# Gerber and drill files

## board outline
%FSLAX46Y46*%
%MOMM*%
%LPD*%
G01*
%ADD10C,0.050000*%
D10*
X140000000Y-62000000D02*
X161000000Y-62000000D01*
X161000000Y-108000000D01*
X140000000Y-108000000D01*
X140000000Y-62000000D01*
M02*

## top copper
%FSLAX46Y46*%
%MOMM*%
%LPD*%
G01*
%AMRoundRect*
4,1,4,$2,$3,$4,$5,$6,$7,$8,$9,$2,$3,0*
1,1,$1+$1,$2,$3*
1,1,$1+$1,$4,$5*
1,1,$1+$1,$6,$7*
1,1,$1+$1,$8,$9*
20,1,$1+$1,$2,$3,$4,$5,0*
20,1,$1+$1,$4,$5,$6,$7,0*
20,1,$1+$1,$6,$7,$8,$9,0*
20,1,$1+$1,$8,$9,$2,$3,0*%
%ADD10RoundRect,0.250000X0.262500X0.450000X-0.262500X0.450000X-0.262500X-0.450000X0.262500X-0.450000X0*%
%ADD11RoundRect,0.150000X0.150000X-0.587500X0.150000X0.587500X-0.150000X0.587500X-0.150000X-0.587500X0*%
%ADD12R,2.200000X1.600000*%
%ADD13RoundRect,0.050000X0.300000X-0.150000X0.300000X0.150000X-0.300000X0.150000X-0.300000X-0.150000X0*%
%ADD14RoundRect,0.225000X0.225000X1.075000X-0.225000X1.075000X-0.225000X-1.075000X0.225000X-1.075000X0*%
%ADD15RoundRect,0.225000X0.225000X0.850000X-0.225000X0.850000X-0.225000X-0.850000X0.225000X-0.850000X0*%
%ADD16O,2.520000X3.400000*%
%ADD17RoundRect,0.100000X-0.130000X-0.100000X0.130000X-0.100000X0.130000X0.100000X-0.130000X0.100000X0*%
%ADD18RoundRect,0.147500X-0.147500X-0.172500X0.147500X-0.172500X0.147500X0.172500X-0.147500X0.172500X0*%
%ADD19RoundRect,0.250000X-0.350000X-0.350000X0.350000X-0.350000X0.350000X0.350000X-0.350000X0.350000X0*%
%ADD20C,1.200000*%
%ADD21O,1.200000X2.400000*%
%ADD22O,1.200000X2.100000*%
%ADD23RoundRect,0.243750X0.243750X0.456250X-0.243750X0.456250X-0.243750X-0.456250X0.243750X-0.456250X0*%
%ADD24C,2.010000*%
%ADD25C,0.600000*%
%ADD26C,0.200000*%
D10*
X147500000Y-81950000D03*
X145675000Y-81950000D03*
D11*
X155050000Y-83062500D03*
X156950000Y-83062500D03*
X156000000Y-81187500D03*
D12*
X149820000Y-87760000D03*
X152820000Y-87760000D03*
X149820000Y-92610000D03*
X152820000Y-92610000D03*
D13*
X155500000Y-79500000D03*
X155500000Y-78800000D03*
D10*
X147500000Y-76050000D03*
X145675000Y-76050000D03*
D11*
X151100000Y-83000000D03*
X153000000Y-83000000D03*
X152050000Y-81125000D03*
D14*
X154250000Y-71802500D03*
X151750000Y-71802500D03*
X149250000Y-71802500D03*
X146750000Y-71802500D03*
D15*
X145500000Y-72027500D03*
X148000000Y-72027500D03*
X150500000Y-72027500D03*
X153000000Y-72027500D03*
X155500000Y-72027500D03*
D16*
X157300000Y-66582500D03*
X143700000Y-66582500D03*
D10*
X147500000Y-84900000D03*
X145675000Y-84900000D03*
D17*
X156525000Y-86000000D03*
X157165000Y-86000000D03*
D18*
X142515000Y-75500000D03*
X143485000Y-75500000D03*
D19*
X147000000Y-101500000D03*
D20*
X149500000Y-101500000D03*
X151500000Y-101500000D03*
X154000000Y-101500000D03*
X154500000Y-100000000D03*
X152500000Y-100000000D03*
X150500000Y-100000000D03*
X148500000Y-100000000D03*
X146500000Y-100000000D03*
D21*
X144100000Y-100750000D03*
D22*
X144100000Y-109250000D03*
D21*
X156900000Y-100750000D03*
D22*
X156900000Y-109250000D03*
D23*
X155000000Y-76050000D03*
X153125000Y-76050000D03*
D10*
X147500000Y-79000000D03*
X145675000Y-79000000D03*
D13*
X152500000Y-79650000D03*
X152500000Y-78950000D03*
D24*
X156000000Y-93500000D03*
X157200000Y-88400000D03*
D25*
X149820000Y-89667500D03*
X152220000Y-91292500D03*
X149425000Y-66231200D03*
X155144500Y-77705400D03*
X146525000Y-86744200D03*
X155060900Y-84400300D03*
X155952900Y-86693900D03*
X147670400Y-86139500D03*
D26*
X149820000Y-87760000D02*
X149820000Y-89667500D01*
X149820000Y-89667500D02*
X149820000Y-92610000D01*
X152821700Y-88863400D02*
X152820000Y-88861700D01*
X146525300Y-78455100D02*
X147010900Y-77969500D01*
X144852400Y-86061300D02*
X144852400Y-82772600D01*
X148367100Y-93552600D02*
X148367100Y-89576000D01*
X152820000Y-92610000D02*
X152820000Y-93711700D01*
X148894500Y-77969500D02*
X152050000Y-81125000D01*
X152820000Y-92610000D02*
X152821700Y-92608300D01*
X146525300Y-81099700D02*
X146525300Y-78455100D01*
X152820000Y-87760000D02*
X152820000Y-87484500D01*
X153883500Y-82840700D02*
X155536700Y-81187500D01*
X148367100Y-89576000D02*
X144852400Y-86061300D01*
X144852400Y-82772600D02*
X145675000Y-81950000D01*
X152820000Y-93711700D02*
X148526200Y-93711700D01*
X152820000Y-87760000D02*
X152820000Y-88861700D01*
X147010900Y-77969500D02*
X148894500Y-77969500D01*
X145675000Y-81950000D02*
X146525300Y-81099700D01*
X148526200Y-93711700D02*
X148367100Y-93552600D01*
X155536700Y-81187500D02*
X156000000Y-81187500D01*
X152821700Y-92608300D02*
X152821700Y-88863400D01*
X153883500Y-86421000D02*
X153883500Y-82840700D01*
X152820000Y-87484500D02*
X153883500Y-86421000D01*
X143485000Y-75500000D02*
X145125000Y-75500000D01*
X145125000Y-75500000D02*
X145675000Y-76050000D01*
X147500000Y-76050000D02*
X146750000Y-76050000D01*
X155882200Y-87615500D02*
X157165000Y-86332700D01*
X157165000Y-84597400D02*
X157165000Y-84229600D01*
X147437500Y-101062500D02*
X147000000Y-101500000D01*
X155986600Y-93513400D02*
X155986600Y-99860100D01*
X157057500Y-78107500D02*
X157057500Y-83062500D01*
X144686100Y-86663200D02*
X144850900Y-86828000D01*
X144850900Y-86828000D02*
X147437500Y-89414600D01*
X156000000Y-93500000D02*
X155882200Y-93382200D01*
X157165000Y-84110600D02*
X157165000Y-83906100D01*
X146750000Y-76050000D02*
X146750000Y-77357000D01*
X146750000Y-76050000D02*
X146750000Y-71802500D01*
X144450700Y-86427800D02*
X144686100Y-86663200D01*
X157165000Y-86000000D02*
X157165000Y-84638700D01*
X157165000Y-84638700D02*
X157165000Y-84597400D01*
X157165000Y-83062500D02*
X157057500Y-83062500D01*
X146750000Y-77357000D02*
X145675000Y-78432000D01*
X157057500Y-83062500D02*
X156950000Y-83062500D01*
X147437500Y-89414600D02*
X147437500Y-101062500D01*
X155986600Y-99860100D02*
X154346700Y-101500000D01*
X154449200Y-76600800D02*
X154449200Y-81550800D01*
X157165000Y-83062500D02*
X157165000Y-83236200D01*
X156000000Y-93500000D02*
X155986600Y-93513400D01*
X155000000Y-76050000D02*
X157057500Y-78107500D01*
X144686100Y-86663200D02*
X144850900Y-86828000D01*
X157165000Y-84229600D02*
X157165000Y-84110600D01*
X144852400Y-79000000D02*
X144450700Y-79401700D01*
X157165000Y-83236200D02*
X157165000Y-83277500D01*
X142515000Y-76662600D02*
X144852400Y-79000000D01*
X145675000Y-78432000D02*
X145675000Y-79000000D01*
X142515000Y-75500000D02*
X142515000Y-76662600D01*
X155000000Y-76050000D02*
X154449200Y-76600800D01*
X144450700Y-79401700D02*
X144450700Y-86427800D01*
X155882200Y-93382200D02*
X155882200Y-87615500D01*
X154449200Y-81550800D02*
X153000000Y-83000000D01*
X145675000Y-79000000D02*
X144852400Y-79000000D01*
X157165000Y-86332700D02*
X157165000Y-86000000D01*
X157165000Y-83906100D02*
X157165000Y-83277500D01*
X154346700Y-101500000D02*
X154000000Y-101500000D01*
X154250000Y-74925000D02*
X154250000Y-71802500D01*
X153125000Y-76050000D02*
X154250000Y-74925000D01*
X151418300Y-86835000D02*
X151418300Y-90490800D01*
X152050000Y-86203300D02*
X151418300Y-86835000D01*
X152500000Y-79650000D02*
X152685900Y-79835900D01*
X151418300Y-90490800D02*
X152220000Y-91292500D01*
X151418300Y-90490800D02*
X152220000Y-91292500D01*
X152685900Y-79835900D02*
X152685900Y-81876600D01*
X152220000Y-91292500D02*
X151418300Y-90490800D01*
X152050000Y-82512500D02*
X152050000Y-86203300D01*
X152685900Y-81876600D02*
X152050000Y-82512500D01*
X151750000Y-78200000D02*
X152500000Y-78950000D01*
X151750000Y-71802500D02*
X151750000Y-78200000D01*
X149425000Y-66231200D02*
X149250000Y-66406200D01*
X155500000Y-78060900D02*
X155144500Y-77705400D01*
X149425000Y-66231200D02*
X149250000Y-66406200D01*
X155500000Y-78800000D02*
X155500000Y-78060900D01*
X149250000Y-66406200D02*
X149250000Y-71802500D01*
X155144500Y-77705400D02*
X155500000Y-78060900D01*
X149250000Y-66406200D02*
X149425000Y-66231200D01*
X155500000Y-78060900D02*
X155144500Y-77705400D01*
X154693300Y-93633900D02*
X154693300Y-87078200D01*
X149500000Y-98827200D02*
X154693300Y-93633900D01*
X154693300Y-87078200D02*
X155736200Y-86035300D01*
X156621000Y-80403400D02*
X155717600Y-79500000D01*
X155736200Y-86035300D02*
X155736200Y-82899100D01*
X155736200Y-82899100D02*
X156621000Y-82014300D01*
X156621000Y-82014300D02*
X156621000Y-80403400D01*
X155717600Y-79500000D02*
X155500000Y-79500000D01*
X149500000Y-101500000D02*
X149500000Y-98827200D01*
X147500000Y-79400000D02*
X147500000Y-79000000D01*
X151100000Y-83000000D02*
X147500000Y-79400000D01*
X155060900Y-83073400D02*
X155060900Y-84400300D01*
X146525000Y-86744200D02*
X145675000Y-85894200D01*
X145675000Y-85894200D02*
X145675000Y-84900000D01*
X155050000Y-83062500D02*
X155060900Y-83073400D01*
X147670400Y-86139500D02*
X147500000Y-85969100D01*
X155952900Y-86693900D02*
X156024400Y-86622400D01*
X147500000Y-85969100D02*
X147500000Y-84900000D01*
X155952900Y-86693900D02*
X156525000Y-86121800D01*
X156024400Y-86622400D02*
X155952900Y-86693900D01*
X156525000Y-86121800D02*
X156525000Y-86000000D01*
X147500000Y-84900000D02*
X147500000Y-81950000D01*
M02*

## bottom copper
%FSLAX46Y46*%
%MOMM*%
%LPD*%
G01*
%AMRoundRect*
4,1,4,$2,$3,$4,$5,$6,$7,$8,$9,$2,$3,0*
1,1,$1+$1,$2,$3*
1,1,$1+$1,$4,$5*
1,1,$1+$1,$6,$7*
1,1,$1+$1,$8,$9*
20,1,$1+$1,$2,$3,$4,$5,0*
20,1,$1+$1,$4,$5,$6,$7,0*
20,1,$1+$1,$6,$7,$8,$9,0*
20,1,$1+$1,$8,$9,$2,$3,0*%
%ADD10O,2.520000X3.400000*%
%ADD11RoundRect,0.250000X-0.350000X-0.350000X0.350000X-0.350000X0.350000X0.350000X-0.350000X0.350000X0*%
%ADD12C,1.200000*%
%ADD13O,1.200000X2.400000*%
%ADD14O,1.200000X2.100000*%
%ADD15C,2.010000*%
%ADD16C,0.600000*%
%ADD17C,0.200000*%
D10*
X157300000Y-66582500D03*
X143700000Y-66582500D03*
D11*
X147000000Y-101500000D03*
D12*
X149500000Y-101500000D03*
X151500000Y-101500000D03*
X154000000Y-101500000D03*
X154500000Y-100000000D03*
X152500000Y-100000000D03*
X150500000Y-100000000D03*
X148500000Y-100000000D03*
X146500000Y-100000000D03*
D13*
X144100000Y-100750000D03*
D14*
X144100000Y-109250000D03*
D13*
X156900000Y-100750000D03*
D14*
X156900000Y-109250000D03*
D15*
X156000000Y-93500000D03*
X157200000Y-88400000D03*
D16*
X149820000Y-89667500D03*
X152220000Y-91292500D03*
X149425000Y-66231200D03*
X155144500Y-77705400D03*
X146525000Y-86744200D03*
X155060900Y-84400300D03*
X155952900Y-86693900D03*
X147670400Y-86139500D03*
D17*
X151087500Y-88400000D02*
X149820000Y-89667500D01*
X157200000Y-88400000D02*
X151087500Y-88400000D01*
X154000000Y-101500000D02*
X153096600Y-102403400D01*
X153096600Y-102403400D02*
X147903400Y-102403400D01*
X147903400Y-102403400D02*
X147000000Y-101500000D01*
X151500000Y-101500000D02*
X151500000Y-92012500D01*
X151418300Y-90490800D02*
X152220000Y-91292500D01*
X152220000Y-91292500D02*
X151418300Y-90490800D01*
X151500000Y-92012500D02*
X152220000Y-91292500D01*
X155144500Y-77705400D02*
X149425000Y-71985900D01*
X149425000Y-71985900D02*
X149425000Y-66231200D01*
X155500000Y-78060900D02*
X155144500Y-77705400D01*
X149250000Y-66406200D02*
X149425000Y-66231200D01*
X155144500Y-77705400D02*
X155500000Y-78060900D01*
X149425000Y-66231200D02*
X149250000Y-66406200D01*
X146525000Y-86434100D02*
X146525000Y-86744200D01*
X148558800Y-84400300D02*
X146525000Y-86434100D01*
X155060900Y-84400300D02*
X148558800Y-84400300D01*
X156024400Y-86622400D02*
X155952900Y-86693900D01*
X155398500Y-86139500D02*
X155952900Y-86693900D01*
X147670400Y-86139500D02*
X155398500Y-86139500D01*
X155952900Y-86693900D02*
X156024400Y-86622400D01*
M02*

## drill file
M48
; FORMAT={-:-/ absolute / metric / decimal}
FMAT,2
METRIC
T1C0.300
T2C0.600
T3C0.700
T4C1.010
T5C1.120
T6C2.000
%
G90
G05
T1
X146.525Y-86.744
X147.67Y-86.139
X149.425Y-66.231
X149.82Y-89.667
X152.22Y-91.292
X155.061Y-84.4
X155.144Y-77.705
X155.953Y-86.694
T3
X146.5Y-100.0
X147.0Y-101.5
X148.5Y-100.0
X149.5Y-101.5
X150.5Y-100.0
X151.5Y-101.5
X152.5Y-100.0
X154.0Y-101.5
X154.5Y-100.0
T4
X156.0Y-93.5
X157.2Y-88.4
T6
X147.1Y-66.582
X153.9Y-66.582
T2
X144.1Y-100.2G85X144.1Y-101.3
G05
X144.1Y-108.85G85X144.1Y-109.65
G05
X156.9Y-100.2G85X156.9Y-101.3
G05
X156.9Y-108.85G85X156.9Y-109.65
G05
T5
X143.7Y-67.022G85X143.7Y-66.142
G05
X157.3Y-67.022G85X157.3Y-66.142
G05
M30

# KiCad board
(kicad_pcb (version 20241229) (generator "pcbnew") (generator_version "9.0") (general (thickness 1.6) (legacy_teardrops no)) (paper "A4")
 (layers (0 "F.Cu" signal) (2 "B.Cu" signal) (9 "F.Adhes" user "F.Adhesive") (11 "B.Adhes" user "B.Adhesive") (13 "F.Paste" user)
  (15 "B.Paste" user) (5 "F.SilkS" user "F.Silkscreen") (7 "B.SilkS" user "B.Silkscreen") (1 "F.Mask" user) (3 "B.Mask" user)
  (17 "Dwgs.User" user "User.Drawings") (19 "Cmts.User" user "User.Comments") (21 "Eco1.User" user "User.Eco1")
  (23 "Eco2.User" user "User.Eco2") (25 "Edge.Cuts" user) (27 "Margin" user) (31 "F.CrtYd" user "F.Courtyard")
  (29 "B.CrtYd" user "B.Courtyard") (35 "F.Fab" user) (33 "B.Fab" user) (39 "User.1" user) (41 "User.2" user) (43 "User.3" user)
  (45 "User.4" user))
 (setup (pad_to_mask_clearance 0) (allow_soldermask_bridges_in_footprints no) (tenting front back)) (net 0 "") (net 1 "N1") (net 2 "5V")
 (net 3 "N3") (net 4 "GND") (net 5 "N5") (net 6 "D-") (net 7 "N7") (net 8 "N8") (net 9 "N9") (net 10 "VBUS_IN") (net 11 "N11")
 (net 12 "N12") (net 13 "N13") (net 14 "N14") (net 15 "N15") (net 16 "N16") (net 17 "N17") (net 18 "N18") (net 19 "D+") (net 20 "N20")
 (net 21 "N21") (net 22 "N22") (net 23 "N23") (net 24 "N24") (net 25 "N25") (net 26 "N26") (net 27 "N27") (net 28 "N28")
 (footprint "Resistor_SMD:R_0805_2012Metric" (layer "F.Cu") (at 146.5875 81.95 180)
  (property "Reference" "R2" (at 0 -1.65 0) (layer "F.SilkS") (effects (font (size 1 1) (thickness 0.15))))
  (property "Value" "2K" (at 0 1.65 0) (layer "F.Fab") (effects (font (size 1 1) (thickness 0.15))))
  (pad "1" smd roundrect (at -0.9125 0 180) (size 1.025 1.4) (layers "F.Cu" "F.Mask" "F.Paste") (roundrect_rratio 0.243902) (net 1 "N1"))
  (pad "2" smd roundrect (at 0.9125 0 180) (size 1.025 1.4) (layers "F.Cu" "F.Mask" "F.Paste") (roundrect_rratio 0.243902) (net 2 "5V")))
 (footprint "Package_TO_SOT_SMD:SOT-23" (layer "F.Cu") (at 156 82.125 90)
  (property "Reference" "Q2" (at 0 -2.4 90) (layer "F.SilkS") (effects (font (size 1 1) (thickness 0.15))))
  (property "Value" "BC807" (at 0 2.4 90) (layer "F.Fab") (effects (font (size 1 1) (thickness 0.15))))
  (pad "1" smd roundrect (at -0.9375 -0.95 90) (size 1.475 0.6) (layers "F.Cu" "F.Mask" "F.Paste") (roundrect_rratio 0.25) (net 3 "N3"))
  (pad "2" smd roundrect (at -0.9375 0.95 90) (size 1.475 0.6) (layers "F.Cu" "F.Mask" "F.Paste") (roundrect_rratio 0.25) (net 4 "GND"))
  (pad "3" smd roundrect (at 0.9375 0 90) (size 1.475 0.6) (layers "F.Cu" "F.Mask" "F.Paste") (roundrect_rratio 0.25) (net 2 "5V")))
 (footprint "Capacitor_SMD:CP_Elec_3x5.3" (layer "F.Cu") (at 151.32 87.76)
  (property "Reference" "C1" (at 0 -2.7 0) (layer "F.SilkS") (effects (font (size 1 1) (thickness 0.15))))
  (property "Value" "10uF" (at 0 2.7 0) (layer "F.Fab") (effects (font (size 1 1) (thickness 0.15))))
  (pad "1" smd rect (at -1.5 0) (size 2.2 1.6) (layers "F.Cu" "F.Mask" "F.Paste") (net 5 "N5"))
  (pad "2" smd rect (at 1.5 0) (size 2.2 1.6) (layers "F.Cu" "F.Mask" "F.Paste") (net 2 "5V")))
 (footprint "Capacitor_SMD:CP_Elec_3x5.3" (layer "F.Cu") (at 151.32 92.61)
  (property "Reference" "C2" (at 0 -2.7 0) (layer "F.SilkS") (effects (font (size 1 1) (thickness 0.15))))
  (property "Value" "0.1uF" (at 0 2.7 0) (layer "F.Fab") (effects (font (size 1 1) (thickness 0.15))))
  (pad "1" smd rect (at -1.5 0) (size 2.2 1.6) (layers "F.Cu" "F.Mask" "F.Paste") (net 5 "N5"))
  (pad "2" smd rect (at 1.5 0) (size 2.2 1.6) (layers "F.Cu" "F.Mask" "F.Paste") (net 2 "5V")))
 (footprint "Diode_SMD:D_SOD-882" (layer "F.Cu") (at 155.5 79.15 90)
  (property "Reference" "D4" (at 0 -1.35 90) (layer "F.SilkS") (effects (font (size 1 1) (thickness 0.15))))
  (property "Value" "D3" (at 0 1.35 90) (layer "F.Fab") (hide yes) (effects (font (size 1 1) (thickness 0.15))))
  (pad "" smd roundrect (at -0.35 0 90) (size 0.3 0.6) (layers "F.Paste") (roundrect_rratio 0.1666666667) (solder_paste_margin -0.05))
  (pad "" smd roundrect (at 0.35 0 90) (size 0.3 0.6) (layers "F.Paste") (roundrect_rratio 0.1666666667) (solder_paste_margin -0.05))
  (pad "1" smd roundrect (at -0.35 0 90) (size 0.4 0.7) (layers "F.Cu" "F.Mask") (roundrect_rratio 0.125) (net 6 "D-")
   (solder_paste_margin -0.05))
  (pad "2" smd roundrect (at 0.35 0 90) (size 0.4 0.7) (layers "F.Cu" "F.Mask") (roundrect_rratio 0.125) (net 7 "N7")
   (solder_paste_margin -0.05)))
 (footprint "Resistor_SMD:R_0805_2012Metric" (layer "F.Cu") (at 146.5875 76.05 180)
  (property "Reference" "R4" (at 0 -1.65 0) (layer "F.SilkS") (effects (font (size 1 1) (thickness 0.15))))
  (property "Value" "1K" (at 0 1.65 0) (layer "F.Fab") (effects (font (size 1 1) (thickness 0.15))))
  (pad "1" smd roundrect (at -0.9125 0 180) (size 1.025 1.4) (layers "F.Cu" "F.Mask" "F.Paste") (roundrect_rratio 0.243902) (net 4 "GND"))
  (pad "2" smd roundrect (at 0.9125 0 180) (size 1.025 1.4) (layers "F.Cu" "F.Mask" "F.Paste") (roundrect_rratio 0.243902) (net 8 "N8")))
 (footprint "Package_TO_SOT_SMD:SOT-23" (layer "F.Cu") (at 152.05 82.0625 90)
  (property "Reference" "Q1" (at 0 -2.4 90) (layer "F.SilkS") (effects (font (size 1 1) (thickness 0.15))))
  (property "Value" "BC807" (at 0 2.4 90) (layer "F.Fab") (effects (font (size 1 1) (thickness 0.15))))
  (pad "1" smd roundrect (at -0.9375 -0.95 90) (size 1.475 0.6) (layers "F.Cu" "F.Mask" "F.Paste") (roundrect_rratio 0.25) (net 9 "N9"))
  (pad "2" smd roundrect (at -0.9375 0.95 90) (size 1.475 0.6) (layers "F.Cu" "F.Mask" "F.Paste") (roundrect_rratio 0.25) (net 4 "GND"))
  (pad "3" smd roundrect (at 0.9375 0 90) (size 1.475 0.6) (layers "F.Cu" "F.Mask" "F.Paste") (roundrect_rratio 0.25) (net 2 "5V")))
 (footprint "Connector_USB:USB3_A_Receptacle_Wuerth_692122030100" (layer "F.Cu") (at 150.5 63.1325 180)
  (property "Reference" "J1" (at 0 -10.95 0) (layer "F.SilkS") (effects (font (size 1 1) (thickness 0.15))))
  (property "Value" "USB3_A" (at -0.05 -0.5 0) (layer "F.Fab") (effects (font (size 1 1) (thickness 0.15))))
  (pad "" np_thru_hole circle (at -3.4 -3.45 180) (size 2 2) (drill 2) (layers "*.Cu" "*.Mask"))
  (pad "" np_thru_hole circle (at 3.4 -3.45 180) (size 2 2) (drill 2) (layers "*.Cu" "*.Mask"))
  (pad "1" smd roundrect (at -3.75 -8.67 180) (size 0.9 2.6) (layers "F.Cu" "F.Mask" "F.Paste") (roundrect_rratio 0.25) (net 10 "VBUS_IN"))
  (pad "2" smd roundrect (at -1.25 -8.67 180) (size 0.9 2.6) (layers "F.Cu" "F.Mask" "F.Paste") (roundrect_rratio 0.25) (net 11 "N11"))
  (pad "3" smd roundrect (at 1.25 -8.67 180) (size 0.9 2.6) (layers "F.Cu" "F.Mask" "F.Paste") (roundrect_rratio 0.25) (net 7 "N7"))
  (pad "4" smd roundrect (at 3.75 -8.67 180) (size 0.9 2.6) (layers "F.Cu" "F.Mask" "F.Paste") (roundrect_rratio 0.25) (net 4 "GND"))
  (pad "5" smd roundrect (at 5 -8.895 180) (size 0.9 2.15) (layers "F.Cu" "F.Mask" "F.Paste") (roundrect_rratio 0.25) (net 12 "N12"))
  (pad "6" smd roundrect (at 2.5 -8.895 180) (size 0.9 2.15) (layers "F.Cu" "F.Mask" "F.Paste") (roundrect_rratio 0.25) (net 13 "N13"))
  (pad "7" smd roundrect (at 0 -8.895 180) (size 0.9 2.15) (layers "F.Cu" "F.Mask" "F.Paste") (roundrect_rratio 0.25) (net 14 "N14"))
  (pad "8" smd roundrect (at -2.5 -8.895 180) (size 0.9 2.15) (layers "F.Cu" "F.Mask" "F.Paste") (roundrect_rratio 0.25) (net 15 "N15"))
  (pad "9" smd roundrect (at -5 -8.895 180) (size 0.9 2.15) (layers "F.Cu" "F.Mask" "F.Paste") (roundrect_rratio 0.25) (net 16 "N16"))
  (pad "10" thru_hole oval (at -6.8 -3.45 180) (size 2.52 3.4) (drill oval 1.12 2) (layers "*.Cu" "*.Mask") (remove_unused_layers no)
   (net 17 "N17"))
  (pad "10" thru_hole oval (at 6.8 -3.45 180) (size 2.52 3.4) (drill oval 1.12 2) (layers "*.Cu" "*.Mask") (remove_unused_layers no)
   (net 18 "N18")))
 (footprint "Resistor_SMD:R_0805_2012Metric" (layer "F.Cu") (at 146.5875 84.9 180)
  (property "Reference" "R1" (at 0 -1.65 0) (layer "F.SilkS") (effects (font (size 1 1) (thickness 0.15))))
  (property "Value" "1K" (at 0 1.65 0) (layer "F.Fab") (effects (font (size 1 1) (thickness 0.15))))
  (pad "1" smd roundrect (at -0.9125 0 180) (size 1.025 1.4) (layers "F.Cu" "F.Mask" "F.Paste") (roundrect_rratio 0.243902) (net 1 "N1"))
  (pad "2" smd roundrect (at 0.9125 0 180) (size 1.025 1.4) (layers "F.Cu" "F.Mask" "F.Paste") (roundrect_rratio 0.243902) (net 3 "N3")))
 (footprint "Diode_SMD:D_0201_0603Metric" (layer "F.Cu") (at 156.845 86)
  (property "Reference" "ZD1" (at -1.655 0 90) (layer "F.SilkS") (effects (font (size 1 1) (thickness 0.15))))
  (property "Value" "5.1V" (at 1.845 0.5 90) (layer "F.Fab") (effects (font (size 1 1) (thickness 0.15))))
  (pad "" smd roundrect (at -0.345 0) (size 0.318 0.36) (layers "F.Paste") (roundrect_rratio 0.25))
  (pad "" smd roundrect (at 0.345 0) (size 0.318 0.36) (layers "F.Paste") (roundrect_rratio 0.25))
  (pad "1" smd roundrect (at -0.32 0) (size 0.46 0.4) (layers "F.Cu" "F.Mask") (roundrect_rratio 0.25) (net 1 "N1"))
  (pad "2" smd roundrect (at 0.32 0) (size 0.46 0.4) (layers "F.Cu" "F.Mask") (roundrect_rratio 0.25) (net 4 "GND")))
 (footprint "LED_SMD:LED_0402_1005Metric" (layer "F.Cu") (at 143 75.5)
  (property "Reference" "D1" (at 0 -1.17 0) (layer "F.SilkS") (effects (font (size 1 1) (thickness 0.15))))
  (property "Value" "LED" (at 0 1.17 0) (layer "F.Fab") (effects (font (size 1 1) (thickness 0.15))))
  (pad "1" smd roundrect (at -0.485 0) (size 0.59 0.64) (layers "F.Cu" "F.Mask" "F.Paste") (roundrect_rratio 0.25) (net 4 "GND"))
  (pad "2" smd roundrect (at 0.485 0) (size 0.59 0.64) (layers "F.Cu" "F.Mask" "F.Paste") (roundrect_rratio 0.25) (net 8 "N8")))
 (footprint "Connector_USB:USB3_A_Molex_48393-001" (layer "F.Cu") (at 147 101.5)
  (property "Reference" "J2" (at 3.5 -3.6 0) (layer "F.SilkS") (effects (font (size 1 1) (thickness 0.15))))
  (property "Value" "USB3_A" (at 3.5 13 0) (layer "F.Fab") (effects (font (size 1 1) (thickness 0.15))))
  (pad "1" thru_hole roundrect (at 0 0) (size 1.2 1.2) (drill 0.7) (layers "*.Cu" "*.Mask") (remove_unused_layers no)
   (roundrect_rratio 0.2083333333) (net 4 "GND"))
  (pad "2" thru_hole circle (at 2.5 0) (size 1.2 1.2) (drill 0.7) (layers "*.Cu" "*.Mask") (remove_unused_layers no) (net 6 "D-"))
  (pad "3" thru_hole circle (at 4.5 0) (size 1.2 1.2) (drill 0.7) (layers "*.Cu" "*.Mask") (remove_unused_layers no) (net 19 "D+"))
  (pad "4" thru_hole circle (at 7 0) (size 1.2 1.2) (drill 0.7) (layers "*.Cu" "*.Mask") (remove_unused_layers no) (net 4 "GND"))
  (pad "5" thru_hole circle (at 7.5 -1.5) (size 1.2 1.2) (drill 0.7) (layers "*.Cu" "*.Mask") (remove_unused_layers no) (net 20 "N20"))
  (pad "6" thru_hole circle (at 5.5 -1.5) (size 1.2 1.2) (drill 0.7) (layers "*.Cu" "*.Mask") (remove_unused_layers no) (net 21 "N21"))
  (pad "7" thru_hole circle (at 3.5 -1.5) (size 1.2 1.2) (drill 0.7) (layers "*.Cu" "*.Mask") (remove_unused_layers no) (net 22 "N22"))
  (pad "8" thru_hole circle (at 1.5 -1.5) (size 1.2 1.2) (drill 0.7) (layers "*.Cu" "*.Mask") (remove_unused_layers no) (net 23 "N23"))
  (pad "9" thru_hole circle (at -0.5 -1.5) (size 1.2 1.2) (drill 0.7) (layers "*.Cu" "*.Mask") (remove_unused_layers no) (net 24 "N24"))
  (pad "10" thru_hole oval (at -2.9 -0.75) (size 1.2 2.4) (drill oval 0.6 1.7) (layers "*.Cu" "*.Mask") (remove_unused_layers no)
   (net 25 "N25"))
  (pad "10" thru_hole oval (at -2.9 7.75) (size 1.2 2.1) (drill oval 0.6 1.4) (layers "*.Cu" "*.Mask") (remove_unused_layers no)
   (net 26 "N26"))
  (pad "10" thru_hole oval (at 9.9 -0.75) (size 1.2 2.4) (drill oval 0.6 1.7) (layers "*.Cu" "*.Mask") (remove_unused_layers no)
   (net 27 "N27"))
  (pad "10" thru_hole oval (at 9.9 7.75) (size 1.2 2.1) (drill oval 0.6 1.4) (layers "*.Cu" "*.Mask") (remove_unused_layers no)
   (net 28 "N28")))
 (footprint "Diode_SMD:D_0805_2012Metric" (layer "F.Cu") (at 154.0625 76.05 180)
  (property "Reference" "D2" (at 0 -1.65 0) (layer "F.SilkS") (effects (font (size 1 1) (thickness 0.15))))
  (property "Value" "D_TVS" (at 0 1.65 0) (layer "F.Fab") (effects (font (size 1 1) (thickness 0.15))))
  (pad "1" smd roundrect (at -0.9375 0 180) (size 0.975 1.4) (layers "F.Cu" "F.Mask" "F.Paste") (roundrect_rratio 0.25) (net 4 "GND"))
  (pad "2" smd roundrect (at 0.9375 0 180) (size 0.975 1.4) (layers "F.Cu" "F.Mask" "F.Paste") (roundrect_rratio 0.25) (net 10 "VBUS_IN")))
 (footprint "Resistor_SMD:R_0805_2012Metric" (layer "F.Cu") (at 146.5875 79 180)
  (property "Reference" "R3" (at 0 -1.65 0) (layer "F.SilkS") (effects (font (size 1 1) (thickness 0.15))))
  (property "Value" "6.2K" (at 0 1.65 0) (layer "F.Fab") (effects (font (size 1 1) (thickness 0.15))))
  (pad "1" smd roundrect (at -0.9125 0 180) (size 1.025 1.4) (layers "F.Cu" "F.Mask" "F.Paste") (roundrect_rratio 0.243902) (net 9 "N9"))
  (pad "2" smd roundrect (at 0.9125 0 180) (size 1.025 1.4) (layers "F.Cu" "F.Mask" "F.Paste") (roundrect_rratio 0.243902) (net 4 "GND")))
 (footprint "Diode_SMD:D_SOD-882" (layer "F.Cu") (at 152.5 79.3 90)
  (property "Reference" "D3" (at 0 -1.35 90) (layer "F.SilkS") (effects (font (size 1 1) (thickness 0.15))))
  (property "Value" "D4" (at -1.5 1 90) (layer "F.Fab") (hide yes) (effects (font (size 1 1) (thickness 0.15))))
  (pad "" smd roundrect (at -0.35 0 90) (size 0.3 0.6) (layers "F.Paste") (roundrect_rratio 0.1666666667) (solder_paste_margin -0.05))
  (pad "" smd roundrect (at 0.35 0 90) (size 0.3 0.6) (layers "F.Paste") (roundrect_rratio 0.1666666667) (solder_paste_margin -0.05))
  (pad "1" smd roundrect (at -0.35 0 90) (size 0.4 0.7) (layers "F.Cu" "F.Mask") (roundrect_rratio 0.125) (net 19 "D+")
   (solder_paste_margin -0.05))
  (pad "2" smd roundrect (at 0.35 0 90) (size 0.4 0.7) (layers "F.Cu" "F.Mask") (roundrect_rratio 0.125) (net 11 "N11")
   (solder_paste_margin -0.05)))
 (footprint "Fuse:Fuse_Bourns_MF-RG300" (layer "F.Cu") (at 156 93.5 90)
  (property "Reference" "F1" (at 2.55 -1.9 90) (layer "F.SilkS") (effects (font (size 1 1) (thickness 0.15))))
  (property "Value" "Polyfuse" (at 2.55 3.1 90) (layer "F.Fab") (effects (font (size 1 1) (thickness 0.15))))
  (pad "1" thru_hole circle (at 0 0 90) (size 2.01 2.01) (drill 1.01) (layers "*.Cu" "*.Mask") (remove_unused_layers no) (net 4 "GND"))
  (pad "2" thru_hole circle (at 5.1 1.2 90) (size 2.01 2.01) (drill 1.01) (layers "*.Cu" "*.Mask") (remove_unused_layers no) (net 5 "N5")))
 (gr_rect (start 140 62) (end 161 108) (stroke (width 0.05) (type default)) (fill no) (layer "Edge.Cuts"))
 (segment (start 149.82 87.76) (end 149.82 89.6675) (width 0.2) (layer "F.Cu") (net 5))
 (segment (start 149.82 89.6675) (end 149.82 92.61) (width 0.2) (layer "F.Cu") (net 5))
 (via (at 149.82 89.6675) (size 0.6) (drill 0.3) (layers "F.Cu" "B.Cu") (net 5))
 (segment (start 151.0875 88.4) (end 149.82 89.6675) (width 0.2) (layer "B.Cu") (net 5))
 (segment (start 157.2 88.4) (end 151.0875 88.4) (width 0.2) (layer "B.Cu") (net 5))
 (segment (start 152.8217 88.8634) (end 152.82 88.8617) (width 0.2) (layer "F.Cu") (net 2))
 (segment (start 146.5253 78.4551) (end 147.0109 77.9695) (width 0.2) (layer "F.Cu") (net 2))
 (segment (start 144.8524 86.0613) (end 144.8524 82.7726) (width 0.2) (layer "F.Cu") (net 2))
 (segment (start 148.3671 93.5526) (end 148.3671 89.576) (width 0.2) (layer "F.Cu") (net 2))
 (segment (start 152.82 92.61) (end 152.82 93.7117) (width 0.2) (layer "F.Cu") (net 2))
 (segment (start 148.8945 77.9695) (end 152.05 81.125) (width 0.2) (layer "F.Cu") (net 2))
 (segment (start 152.82 92.61) (end 152.8217 92.6083) (width 0.2) (layer "F.Cu") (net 2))
 (segment (start 146.5253 81.0997) (end 146.5253 78.4551) (width 0.2) (layer "F.Cu") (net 2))
 (segment (start 152.82 87.76) (end 152.82 87.4845) (width 0.2) (layer "F.Cu") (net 2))
 (segment (start 153.8835 82.8407) (end 155.5367 81.1875) (width 0.2) (layer "F.Cu") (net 2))
 (segment (start 148.3671 89.576) (end 144.8524 86.0613) (width 0.2) (layer "F.Cu") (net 2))
 (segment (start 144.8524 82.7726) (end 145.675 81.95) (width 0.2) (layer "F.Cu") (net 2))
 (segment (start 152.82 93.7117) (end 148.5262 93.7117) (width 0.2) (layer "F.Cu") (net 2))
 (segment (start 152.82 87.76) (end 152.82 88.8617) (width 0.2) (layer "F.Cu") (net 2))
 (segment (start 147.0109 77.9695) (end 148.8945 77.9695) (width 0.2) (layer "F.Cu") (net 2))
 (segment (start 145.675 81.95) (end 146.5253 81.0997) (width 0.2) (layer "F.Cu") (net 2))
 (segment (start 148.5262 93.7117) (end 148.3671 93.5526) (width 0.2) (layer "F.Cu") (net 2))
 (segment (start 155.5367 81.1875) (end 156 81.1875) (width 0.2) (layer "F.Cu") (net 2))
 (segment (start 152.8217 92.6083) (end 152.8217 88.8634) (width 0.2) (layer "F.Cu") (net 2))
 (segment (start 153.8835 86.421) (end 153.8835 82.8407) (width 0.2) (layer "F.Cu") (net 2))
 (segment (start 152.82 87.4845) (end 153.8835 86.421) (width 0.2) (layer "F.Cu") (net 2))
 (segment (start 143.485 75.5) (end 145.125 75.5) (width 0.2) (layer "F.Cu") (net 8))
 (segment (start 145.125 75.5) (end 145.675 76.05) (width 0.2) (layer "F.Cu") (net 8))
 (segment (start 147.5 76.05) (end 146.75 76.05) (width 0.2) (layer "F.Cu") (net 4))
 (segment (start 155.8822 87.6155) (end 157.165 86.3327) (width 0.2) (layer "F.Cu") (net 4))
 (segment (start 157.165 84.5974) (end 157.165 84.2296) (width 0.2) (layer "F.Cu") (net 4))
 (segment (start 147.4375 101.0625) (end 147 101.5) (width 0.2) (layer "F.Cu") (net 4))
 (segment (start 155.9866 93.5134) (end 155.9866 99.8601) (width 0.2) (layer "F.Cu") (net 4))
 (segment (start 157.0575 78.1075) (end 157.0575 83.0625) (width 0.2) (layer "F.Cu") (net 4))
 (segment (start 144.6861 86.6632) (end 144.8509 86.828) (width 0.2) (layer "F.Cu") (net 4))
 (segment (start 144.8509 86.828) (end 147.4375 89.4146) (width 0.2) (layer "F.Cu") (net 4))
 (segment (start 156 93.5) (end 155.8822 93.3822) (width 0.2) (layer "F.Cu") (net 4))
 (segment (start 157.165 84.1106) (end 157.165 83.9061) (width 0.2) (layer "F.Cu") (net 4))
 (segment (start 146.75 76.05) (end 146.75 77.357) (width 0.2) (layer "F.Cu") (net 4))
 (segment (start 146.75 76.05) (end 146.75 71.8025) (width 0.2) (layer "F.Cu") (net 4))
 (segment (start 144.4507 86.4278) (end 144.6861 86.6632) (width 0.2) (layer "F.Cu") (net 4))
 (segment (start 157.165 86) (end 157.165 84.6387) (width 0.2) (layer "F.Cu") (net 4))
 (segment (start 157.165 84.6387) (end 157.165 84.5974) (width 0.2) (layer "F.Cu") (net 4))
 (segment (start 157.165 83.0625) (end 157.0575 83.0625) (width 0.2) (layer "F.Cu") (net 4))
 (segment (start 146.75 77.357) (end 145.675 78.432) (width 0.2) (layer "F.Cu") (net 4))
 (segment (start 157.0575 83.0625) (end 156.95 83.0625) (width 0.2) (layer "F.Cu") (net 4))
 (segment (start 147.4375 89.4146) (end 147.4375 101.0625) (width 0.2) (layer "F.Cu") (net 4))
 (segment (start 155.9866 99.8601) (end 154.3467 101.5) (width 0.2) (layer "F.Cu") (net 4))
 (segment (start 154.4492 76.6008) (end 154.4492 81.5508) (width 0.2) (layer "F.Cu") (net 4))
 (segment (start 157.165 83.0625) (end 157.165 83.2362) (width 0.2) (layer "F.Cu") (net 4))
 (segment (start 156 93.5) (end 155.9866 93.5134) (width 0.2) (layer "F.Cu") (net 4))
 (segment (start 155 76.05) (end 157.0575 78.1075) (width 0.2) (layer "F.Cu") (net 4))
 (segment (start 144.6861 86.6632) (end 144.8509 86.828) (width 0.2) (layer "F.Cu") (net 4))
 (segment (start 157.165 84.2296) (end 157.165 84.1106) (width 0.2) (layer "F.Cu") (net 4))
 (segment (start 144.8524 79) (end 144.4507 79.4017) (width 0.2) (layer "F.Cu") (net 4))
 (segment (start 157.165 83.2362) (end 157.165 83.2775) (width 0.2) (layer "F.Cu") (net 4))
 (segment (start 142.515 76.6626) (end 144.8524 79) (width 0.2) (layer "F.Cu") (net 4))
 (segment (start 145.675 78.432) (end 145.675 79) (width 0.2) (layer "F.Cu") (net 4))
 (segment (start 142.515 75.5) (end 142.515 76.6626) (width 0.2) (layer "F.Cu") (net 4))
 (segment (start 155 76.05) (end 154.4492 76.6008) (width 0.2) (layer "F.Cu") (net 4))
 (segment (start 144.4507 79.4017) (end 144.4507 86.4278) (width 0.2) (layer "F.Cu") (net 4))
 (segment (start 155.8822 93.3822) (end 155.8822 87.6155) (width 0.2) (layer "F.Cu") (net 4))
 (segment (start 154.4492 81.5508) (end 153 83) (width 0.2) (layer "F.Cu") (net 4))
 (segment (start 145.675 79) (end 144.8524 79) (width 0.2) (layer "F.Cu") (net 4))
 (segment (start 157.165 86.3327) (end 157.165 86) (width 0.2) (layer "F.Cu") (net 4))
 (segment (start 157.165 83.9061) (end 157.165 83.2775) (width 0.2) (layer "F.Cu") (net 4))
 (segment (start 154.3467 101.5) (end 154 101.5) (width 0.2) (layer "F.Cu") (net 4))
 (segment (start 154 101.5) (end 153.0966 102.4034) (width 0.2) (layer "B.Cu") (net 4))
 (segment (start 153.0966 102.4034) (end 147.9034 102.4034) (width 0.2) (layer "B.Cu") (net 4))
 (segment (start 147.9034 102.4034) (end 147 101.5) (width 0.2) (layer "B.Cu") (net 4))
 (segment (start 154.25 74.925) (end 154.25 71.8025) (width 0.2) (layer "F.Cu") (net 10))
 (segment (start 153.125 76.05) (end 154.25 74.925) (width 0.2) (layer "F.Cu") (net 10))
 (segment (start 151.4183 86.835) (end 151.4183 90.4908) (width 0.2) (layer "F.Cu") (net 19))
 (segment (start 152.05 86.2033) (end 151.4183 86.835) (width 0.2) (layer "F.Cu") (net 19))
 (segment (start 152.5 79.65) (end 152.6859 79.8359) (width 0.2) (layer "F.Cu") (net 19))
 (segment (start 151.4183 90.4908) (end 152.22 91.2925) (width 0.2) (layer "F.Cu") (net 19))
 (segment (start 151.4183 90.4908) (end 152.22 91.2925) (width 0.2) (layer "F.Cu") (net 19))
 (segment (start 152.6859 79.8359) (end 152.6859 81.8766) (width 0.2) (layer "F.Cu") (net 19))
 (segment (start 152.22 91.2925) (end 151.4183 90.4908) (width 0.2) (layer "F.Cu") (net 19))
 (segment (start 152.05 82.5125) (end 152.05 86.2033) (width 0.2) (layer "F.Cu") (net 19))
 (segment (start 152.6859 81.8766) (end 152.05 82.5125) (width 0.2) (layer "F.Cu") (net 19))
 (via (at 152.22 91.2925) (size 0.6) (drill 0.3) (layers "F.Cu" "B.Cu") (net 19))
 (segment (start 151.5 101.5) (end 151.5 92.0125) (width 0.2) (layer "B.Cu") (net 19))
 (segment (start 151.4183 90.4908) (end 152.22 91.2925) (width 0.2) (layer "B.Cu") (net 19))
 (segment (start 152.22 91.2925) (end 151.4183 90.4908) (width 0.2) (layer "B.Cu") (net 19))
 (segment (start 151.5 92.0125) (end 152.22 91.2925) (width 0.2) (layer "B.Cu") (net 19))
 (segment (start 151.75 78.2) (end 152.5 78.95) (width 0.2) (layer "F.Cu") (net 11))
 (segment (start 151.75 71.8025) (end 151.75 78.2) (width 0.2) (layer "F.Cu") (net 11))
 (segment (start 149.425 66.2312) (end 149.25 66.4062) (width 0.2) (layer "F.Cu") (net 7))
 (segment (start 155.5 78.0609) (end 155.1445 77.7054) (width 0.2) (layer "F.Cu") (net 7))
 (segment (start 149.425 66.2312) (end 149.25 66.4062) (width 0.2) (layer "F.Cu") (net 7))
 (segment (start 155.5 78.8) (end 155.5 78.0609) (width 0.2) (layer "F.Cu") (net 7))
 (segment (start 149.25 66.4062) (end 149.25 71.8025) (width 0.2) (layer "F.Cu") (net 7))
 (segment (start 155.1445 77.7054) (end 155.5 78.0609) (width 0.2) (layer "F.Cu") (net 7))
 (segment (start 149.25 66.4062) (end 149.425 66.2312) (width 0.2) (layer "F.Cu") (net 7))
 (segment (start 155.5 78.0609) (end 155.1445 77.7054) (width 0.2) (layer "F.Cu") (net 7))
 (via (at 149.425 66.2312) (size 0.6) (drill 0.3) (layers "F.Cu" "B.Cu") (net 7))
 (via (at 155.1445 77.7054) (size 0.6) (drill 0.3) (layers "F.Cu" "B.Cu") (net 7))
 (segment (start 155.1445 77.7054) (end 149.425 71.9859) (width 0.2) (layer "B.Cu") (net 7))
 (segment (start 149.425 71.9859) (end 149.425 66.2312) (width 0.2) (layer "B.Cu") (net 7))
 (segment (start 155.5 78.0609) (end 155.1445 77.7054) (width 0.2) (layer "B.Cu") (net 7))
 (segment (start 149.25 66.4062) (end 149.425 66.2312) (width 0.2) (layer "B.Cu") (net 7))
 (segment (start 155.1445 77.7054) (end 155.5 78.0609) (width 0.2) (layer "B.Cu") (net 7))
 (segment (start 149.425 66.2312) (end 149.25 66.4062) (width 0.2) (layer "B.Cu") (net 7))
 (segment (start 154.6933 93.6339) (end 154.6933 87.0782) (width 0.2) (layer "F.Cu") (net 6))
 (segment (start 149.5 98.8272) (end 154.6933 93.6339) (width 0.2) (layer "F.Cu") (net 6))
 (segment (start 154.6933 87.0782) (end 155.7362 86.0353) (width 0.2) (layer "F.Cu") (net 6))
 (segment (start 156.621 80.4034) (end 155.7176 79.5) (width 0.2) (layer "F.Cu") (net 6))
 (segment (start 155.7362 86.0353) (end 155.7362 82.8991) (width 0.2) (layer "F.Cu") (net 6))
 (segment (start 155.7362 82.8991) (end 156.621 82.0143) (width 0.2) (layer "F.Cu") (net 6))
 (segment (start 156.621 82.0143) (end 156.621 80.4034) (width 0.2) (layer "F.Cu") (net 6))
 (segment (start 155.7176 79.5) (end 155.5 79.5) (width 0.2) (layer "F.Cu") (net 6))
 (segment (start 149.5 101.5) (end 149.5 98.8272) (width 0.2) (layer "F.Cu") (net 6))
 (segment (start 147.5 79.4) (end 147.5 79) (width 0.2) (layer "F.Cu") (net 9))
 (segment (start 151.1 83) (end 147.5 79.4) (width 0.2) (layer "F.Cu") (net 9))
 (segment (start 155.0609 83.0734) (end 155.0609 84.4003) (width 0.2) (layer "F.Cu") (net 3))
 (segment (start 146.525 86.7442) (end 145.675 85.8942) (width 0.2) (layer "F.Cu") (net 3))
 (segment (start 145.675 85.8942) (end 145.675 84.9) (width 0.2) (layer "F.Cu") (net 3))
 (segment (start 155.05 83.0625) (end 155.0609 83.0734) (width 0.2) (layer "F.Cu") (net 3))
 (via (at 146.525 86.7442) (size 0.6) (drill 0.3) (layers "F.Cu" "B.Cu") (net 3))
 (via (at 155.0609 84.4003) (size 0.6) (drill 0.3) (layers "F.Cu" "B.Cu") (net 3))
 (segment (start 146.525 86.4341) (end 146.525 86.7442) (width 0.2) (layer "B.Cu") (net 3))
 (segment (start 148.5588 84.4003) (end 146.525 86.4341) (width 0.2) (layer "B.Cu") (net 3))
 (segment (start 155.0609 84.4003) (end 148.5588 84.4003) (width 0.2) (layer "B.Cu") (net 3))
 (segment (start 147.6704 86.1395) (end 147.5 85.9691) (width 0.2) (layer "F.Cu") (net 1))
 (segment (start 155.9529 86.6939) (end 156.0244 86.6224) (width 0.2) (layer "F.Cu") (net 1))
 (segment (start 147.5 85.9691) (end 147.5 84.9) (width 0.2) (layer "F.Cu") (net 1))
 (segment (start 155.9529 86.6939) (end 156.525 86.1218) (width 0.2) (layer "F.Cu") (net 1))
 (segment (start 156.0244 86.6224) (end 155.9529 86.6939) (width 0.2) (layer "F.Cu") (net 1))
 (segment (start 156.525 86.1218) (end 156.525 86) (width 0.2) (layer "F.Cu") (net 1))
 (segment (start 147.5 84.9) (end 147.5 81.95) (width 0.2) (layer "F.Cu") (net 1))
 (via (at 155.9529 86.6939) (size 0.6) (drill 0.3) (layers "F.Cu" "B.Cu") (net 1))
 (via (at 147.6704 86.1395) (size 0.6) (drill 0.3) (layers "F.Cu" "B.Cu") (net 1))
 (segment (start 156.0244 86.6224) (end 155.9529 86.6939) (width 0.2) (layer "B.Cu") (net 1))
 (segment (start 155.3985 86.1395) (end 155.9529 86.6939) (width 0.2) (layer "B.Cu") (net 1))
 (segment (start 147.6704 86.1395) (end 155.3985 86.1395) (width 0.2) (layer "B.Cu") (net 1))
 (segment (start 155.9529 86.6939) (end 156.0244 86.6224) (width 0.2) (layer "B.Cu") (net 1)))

